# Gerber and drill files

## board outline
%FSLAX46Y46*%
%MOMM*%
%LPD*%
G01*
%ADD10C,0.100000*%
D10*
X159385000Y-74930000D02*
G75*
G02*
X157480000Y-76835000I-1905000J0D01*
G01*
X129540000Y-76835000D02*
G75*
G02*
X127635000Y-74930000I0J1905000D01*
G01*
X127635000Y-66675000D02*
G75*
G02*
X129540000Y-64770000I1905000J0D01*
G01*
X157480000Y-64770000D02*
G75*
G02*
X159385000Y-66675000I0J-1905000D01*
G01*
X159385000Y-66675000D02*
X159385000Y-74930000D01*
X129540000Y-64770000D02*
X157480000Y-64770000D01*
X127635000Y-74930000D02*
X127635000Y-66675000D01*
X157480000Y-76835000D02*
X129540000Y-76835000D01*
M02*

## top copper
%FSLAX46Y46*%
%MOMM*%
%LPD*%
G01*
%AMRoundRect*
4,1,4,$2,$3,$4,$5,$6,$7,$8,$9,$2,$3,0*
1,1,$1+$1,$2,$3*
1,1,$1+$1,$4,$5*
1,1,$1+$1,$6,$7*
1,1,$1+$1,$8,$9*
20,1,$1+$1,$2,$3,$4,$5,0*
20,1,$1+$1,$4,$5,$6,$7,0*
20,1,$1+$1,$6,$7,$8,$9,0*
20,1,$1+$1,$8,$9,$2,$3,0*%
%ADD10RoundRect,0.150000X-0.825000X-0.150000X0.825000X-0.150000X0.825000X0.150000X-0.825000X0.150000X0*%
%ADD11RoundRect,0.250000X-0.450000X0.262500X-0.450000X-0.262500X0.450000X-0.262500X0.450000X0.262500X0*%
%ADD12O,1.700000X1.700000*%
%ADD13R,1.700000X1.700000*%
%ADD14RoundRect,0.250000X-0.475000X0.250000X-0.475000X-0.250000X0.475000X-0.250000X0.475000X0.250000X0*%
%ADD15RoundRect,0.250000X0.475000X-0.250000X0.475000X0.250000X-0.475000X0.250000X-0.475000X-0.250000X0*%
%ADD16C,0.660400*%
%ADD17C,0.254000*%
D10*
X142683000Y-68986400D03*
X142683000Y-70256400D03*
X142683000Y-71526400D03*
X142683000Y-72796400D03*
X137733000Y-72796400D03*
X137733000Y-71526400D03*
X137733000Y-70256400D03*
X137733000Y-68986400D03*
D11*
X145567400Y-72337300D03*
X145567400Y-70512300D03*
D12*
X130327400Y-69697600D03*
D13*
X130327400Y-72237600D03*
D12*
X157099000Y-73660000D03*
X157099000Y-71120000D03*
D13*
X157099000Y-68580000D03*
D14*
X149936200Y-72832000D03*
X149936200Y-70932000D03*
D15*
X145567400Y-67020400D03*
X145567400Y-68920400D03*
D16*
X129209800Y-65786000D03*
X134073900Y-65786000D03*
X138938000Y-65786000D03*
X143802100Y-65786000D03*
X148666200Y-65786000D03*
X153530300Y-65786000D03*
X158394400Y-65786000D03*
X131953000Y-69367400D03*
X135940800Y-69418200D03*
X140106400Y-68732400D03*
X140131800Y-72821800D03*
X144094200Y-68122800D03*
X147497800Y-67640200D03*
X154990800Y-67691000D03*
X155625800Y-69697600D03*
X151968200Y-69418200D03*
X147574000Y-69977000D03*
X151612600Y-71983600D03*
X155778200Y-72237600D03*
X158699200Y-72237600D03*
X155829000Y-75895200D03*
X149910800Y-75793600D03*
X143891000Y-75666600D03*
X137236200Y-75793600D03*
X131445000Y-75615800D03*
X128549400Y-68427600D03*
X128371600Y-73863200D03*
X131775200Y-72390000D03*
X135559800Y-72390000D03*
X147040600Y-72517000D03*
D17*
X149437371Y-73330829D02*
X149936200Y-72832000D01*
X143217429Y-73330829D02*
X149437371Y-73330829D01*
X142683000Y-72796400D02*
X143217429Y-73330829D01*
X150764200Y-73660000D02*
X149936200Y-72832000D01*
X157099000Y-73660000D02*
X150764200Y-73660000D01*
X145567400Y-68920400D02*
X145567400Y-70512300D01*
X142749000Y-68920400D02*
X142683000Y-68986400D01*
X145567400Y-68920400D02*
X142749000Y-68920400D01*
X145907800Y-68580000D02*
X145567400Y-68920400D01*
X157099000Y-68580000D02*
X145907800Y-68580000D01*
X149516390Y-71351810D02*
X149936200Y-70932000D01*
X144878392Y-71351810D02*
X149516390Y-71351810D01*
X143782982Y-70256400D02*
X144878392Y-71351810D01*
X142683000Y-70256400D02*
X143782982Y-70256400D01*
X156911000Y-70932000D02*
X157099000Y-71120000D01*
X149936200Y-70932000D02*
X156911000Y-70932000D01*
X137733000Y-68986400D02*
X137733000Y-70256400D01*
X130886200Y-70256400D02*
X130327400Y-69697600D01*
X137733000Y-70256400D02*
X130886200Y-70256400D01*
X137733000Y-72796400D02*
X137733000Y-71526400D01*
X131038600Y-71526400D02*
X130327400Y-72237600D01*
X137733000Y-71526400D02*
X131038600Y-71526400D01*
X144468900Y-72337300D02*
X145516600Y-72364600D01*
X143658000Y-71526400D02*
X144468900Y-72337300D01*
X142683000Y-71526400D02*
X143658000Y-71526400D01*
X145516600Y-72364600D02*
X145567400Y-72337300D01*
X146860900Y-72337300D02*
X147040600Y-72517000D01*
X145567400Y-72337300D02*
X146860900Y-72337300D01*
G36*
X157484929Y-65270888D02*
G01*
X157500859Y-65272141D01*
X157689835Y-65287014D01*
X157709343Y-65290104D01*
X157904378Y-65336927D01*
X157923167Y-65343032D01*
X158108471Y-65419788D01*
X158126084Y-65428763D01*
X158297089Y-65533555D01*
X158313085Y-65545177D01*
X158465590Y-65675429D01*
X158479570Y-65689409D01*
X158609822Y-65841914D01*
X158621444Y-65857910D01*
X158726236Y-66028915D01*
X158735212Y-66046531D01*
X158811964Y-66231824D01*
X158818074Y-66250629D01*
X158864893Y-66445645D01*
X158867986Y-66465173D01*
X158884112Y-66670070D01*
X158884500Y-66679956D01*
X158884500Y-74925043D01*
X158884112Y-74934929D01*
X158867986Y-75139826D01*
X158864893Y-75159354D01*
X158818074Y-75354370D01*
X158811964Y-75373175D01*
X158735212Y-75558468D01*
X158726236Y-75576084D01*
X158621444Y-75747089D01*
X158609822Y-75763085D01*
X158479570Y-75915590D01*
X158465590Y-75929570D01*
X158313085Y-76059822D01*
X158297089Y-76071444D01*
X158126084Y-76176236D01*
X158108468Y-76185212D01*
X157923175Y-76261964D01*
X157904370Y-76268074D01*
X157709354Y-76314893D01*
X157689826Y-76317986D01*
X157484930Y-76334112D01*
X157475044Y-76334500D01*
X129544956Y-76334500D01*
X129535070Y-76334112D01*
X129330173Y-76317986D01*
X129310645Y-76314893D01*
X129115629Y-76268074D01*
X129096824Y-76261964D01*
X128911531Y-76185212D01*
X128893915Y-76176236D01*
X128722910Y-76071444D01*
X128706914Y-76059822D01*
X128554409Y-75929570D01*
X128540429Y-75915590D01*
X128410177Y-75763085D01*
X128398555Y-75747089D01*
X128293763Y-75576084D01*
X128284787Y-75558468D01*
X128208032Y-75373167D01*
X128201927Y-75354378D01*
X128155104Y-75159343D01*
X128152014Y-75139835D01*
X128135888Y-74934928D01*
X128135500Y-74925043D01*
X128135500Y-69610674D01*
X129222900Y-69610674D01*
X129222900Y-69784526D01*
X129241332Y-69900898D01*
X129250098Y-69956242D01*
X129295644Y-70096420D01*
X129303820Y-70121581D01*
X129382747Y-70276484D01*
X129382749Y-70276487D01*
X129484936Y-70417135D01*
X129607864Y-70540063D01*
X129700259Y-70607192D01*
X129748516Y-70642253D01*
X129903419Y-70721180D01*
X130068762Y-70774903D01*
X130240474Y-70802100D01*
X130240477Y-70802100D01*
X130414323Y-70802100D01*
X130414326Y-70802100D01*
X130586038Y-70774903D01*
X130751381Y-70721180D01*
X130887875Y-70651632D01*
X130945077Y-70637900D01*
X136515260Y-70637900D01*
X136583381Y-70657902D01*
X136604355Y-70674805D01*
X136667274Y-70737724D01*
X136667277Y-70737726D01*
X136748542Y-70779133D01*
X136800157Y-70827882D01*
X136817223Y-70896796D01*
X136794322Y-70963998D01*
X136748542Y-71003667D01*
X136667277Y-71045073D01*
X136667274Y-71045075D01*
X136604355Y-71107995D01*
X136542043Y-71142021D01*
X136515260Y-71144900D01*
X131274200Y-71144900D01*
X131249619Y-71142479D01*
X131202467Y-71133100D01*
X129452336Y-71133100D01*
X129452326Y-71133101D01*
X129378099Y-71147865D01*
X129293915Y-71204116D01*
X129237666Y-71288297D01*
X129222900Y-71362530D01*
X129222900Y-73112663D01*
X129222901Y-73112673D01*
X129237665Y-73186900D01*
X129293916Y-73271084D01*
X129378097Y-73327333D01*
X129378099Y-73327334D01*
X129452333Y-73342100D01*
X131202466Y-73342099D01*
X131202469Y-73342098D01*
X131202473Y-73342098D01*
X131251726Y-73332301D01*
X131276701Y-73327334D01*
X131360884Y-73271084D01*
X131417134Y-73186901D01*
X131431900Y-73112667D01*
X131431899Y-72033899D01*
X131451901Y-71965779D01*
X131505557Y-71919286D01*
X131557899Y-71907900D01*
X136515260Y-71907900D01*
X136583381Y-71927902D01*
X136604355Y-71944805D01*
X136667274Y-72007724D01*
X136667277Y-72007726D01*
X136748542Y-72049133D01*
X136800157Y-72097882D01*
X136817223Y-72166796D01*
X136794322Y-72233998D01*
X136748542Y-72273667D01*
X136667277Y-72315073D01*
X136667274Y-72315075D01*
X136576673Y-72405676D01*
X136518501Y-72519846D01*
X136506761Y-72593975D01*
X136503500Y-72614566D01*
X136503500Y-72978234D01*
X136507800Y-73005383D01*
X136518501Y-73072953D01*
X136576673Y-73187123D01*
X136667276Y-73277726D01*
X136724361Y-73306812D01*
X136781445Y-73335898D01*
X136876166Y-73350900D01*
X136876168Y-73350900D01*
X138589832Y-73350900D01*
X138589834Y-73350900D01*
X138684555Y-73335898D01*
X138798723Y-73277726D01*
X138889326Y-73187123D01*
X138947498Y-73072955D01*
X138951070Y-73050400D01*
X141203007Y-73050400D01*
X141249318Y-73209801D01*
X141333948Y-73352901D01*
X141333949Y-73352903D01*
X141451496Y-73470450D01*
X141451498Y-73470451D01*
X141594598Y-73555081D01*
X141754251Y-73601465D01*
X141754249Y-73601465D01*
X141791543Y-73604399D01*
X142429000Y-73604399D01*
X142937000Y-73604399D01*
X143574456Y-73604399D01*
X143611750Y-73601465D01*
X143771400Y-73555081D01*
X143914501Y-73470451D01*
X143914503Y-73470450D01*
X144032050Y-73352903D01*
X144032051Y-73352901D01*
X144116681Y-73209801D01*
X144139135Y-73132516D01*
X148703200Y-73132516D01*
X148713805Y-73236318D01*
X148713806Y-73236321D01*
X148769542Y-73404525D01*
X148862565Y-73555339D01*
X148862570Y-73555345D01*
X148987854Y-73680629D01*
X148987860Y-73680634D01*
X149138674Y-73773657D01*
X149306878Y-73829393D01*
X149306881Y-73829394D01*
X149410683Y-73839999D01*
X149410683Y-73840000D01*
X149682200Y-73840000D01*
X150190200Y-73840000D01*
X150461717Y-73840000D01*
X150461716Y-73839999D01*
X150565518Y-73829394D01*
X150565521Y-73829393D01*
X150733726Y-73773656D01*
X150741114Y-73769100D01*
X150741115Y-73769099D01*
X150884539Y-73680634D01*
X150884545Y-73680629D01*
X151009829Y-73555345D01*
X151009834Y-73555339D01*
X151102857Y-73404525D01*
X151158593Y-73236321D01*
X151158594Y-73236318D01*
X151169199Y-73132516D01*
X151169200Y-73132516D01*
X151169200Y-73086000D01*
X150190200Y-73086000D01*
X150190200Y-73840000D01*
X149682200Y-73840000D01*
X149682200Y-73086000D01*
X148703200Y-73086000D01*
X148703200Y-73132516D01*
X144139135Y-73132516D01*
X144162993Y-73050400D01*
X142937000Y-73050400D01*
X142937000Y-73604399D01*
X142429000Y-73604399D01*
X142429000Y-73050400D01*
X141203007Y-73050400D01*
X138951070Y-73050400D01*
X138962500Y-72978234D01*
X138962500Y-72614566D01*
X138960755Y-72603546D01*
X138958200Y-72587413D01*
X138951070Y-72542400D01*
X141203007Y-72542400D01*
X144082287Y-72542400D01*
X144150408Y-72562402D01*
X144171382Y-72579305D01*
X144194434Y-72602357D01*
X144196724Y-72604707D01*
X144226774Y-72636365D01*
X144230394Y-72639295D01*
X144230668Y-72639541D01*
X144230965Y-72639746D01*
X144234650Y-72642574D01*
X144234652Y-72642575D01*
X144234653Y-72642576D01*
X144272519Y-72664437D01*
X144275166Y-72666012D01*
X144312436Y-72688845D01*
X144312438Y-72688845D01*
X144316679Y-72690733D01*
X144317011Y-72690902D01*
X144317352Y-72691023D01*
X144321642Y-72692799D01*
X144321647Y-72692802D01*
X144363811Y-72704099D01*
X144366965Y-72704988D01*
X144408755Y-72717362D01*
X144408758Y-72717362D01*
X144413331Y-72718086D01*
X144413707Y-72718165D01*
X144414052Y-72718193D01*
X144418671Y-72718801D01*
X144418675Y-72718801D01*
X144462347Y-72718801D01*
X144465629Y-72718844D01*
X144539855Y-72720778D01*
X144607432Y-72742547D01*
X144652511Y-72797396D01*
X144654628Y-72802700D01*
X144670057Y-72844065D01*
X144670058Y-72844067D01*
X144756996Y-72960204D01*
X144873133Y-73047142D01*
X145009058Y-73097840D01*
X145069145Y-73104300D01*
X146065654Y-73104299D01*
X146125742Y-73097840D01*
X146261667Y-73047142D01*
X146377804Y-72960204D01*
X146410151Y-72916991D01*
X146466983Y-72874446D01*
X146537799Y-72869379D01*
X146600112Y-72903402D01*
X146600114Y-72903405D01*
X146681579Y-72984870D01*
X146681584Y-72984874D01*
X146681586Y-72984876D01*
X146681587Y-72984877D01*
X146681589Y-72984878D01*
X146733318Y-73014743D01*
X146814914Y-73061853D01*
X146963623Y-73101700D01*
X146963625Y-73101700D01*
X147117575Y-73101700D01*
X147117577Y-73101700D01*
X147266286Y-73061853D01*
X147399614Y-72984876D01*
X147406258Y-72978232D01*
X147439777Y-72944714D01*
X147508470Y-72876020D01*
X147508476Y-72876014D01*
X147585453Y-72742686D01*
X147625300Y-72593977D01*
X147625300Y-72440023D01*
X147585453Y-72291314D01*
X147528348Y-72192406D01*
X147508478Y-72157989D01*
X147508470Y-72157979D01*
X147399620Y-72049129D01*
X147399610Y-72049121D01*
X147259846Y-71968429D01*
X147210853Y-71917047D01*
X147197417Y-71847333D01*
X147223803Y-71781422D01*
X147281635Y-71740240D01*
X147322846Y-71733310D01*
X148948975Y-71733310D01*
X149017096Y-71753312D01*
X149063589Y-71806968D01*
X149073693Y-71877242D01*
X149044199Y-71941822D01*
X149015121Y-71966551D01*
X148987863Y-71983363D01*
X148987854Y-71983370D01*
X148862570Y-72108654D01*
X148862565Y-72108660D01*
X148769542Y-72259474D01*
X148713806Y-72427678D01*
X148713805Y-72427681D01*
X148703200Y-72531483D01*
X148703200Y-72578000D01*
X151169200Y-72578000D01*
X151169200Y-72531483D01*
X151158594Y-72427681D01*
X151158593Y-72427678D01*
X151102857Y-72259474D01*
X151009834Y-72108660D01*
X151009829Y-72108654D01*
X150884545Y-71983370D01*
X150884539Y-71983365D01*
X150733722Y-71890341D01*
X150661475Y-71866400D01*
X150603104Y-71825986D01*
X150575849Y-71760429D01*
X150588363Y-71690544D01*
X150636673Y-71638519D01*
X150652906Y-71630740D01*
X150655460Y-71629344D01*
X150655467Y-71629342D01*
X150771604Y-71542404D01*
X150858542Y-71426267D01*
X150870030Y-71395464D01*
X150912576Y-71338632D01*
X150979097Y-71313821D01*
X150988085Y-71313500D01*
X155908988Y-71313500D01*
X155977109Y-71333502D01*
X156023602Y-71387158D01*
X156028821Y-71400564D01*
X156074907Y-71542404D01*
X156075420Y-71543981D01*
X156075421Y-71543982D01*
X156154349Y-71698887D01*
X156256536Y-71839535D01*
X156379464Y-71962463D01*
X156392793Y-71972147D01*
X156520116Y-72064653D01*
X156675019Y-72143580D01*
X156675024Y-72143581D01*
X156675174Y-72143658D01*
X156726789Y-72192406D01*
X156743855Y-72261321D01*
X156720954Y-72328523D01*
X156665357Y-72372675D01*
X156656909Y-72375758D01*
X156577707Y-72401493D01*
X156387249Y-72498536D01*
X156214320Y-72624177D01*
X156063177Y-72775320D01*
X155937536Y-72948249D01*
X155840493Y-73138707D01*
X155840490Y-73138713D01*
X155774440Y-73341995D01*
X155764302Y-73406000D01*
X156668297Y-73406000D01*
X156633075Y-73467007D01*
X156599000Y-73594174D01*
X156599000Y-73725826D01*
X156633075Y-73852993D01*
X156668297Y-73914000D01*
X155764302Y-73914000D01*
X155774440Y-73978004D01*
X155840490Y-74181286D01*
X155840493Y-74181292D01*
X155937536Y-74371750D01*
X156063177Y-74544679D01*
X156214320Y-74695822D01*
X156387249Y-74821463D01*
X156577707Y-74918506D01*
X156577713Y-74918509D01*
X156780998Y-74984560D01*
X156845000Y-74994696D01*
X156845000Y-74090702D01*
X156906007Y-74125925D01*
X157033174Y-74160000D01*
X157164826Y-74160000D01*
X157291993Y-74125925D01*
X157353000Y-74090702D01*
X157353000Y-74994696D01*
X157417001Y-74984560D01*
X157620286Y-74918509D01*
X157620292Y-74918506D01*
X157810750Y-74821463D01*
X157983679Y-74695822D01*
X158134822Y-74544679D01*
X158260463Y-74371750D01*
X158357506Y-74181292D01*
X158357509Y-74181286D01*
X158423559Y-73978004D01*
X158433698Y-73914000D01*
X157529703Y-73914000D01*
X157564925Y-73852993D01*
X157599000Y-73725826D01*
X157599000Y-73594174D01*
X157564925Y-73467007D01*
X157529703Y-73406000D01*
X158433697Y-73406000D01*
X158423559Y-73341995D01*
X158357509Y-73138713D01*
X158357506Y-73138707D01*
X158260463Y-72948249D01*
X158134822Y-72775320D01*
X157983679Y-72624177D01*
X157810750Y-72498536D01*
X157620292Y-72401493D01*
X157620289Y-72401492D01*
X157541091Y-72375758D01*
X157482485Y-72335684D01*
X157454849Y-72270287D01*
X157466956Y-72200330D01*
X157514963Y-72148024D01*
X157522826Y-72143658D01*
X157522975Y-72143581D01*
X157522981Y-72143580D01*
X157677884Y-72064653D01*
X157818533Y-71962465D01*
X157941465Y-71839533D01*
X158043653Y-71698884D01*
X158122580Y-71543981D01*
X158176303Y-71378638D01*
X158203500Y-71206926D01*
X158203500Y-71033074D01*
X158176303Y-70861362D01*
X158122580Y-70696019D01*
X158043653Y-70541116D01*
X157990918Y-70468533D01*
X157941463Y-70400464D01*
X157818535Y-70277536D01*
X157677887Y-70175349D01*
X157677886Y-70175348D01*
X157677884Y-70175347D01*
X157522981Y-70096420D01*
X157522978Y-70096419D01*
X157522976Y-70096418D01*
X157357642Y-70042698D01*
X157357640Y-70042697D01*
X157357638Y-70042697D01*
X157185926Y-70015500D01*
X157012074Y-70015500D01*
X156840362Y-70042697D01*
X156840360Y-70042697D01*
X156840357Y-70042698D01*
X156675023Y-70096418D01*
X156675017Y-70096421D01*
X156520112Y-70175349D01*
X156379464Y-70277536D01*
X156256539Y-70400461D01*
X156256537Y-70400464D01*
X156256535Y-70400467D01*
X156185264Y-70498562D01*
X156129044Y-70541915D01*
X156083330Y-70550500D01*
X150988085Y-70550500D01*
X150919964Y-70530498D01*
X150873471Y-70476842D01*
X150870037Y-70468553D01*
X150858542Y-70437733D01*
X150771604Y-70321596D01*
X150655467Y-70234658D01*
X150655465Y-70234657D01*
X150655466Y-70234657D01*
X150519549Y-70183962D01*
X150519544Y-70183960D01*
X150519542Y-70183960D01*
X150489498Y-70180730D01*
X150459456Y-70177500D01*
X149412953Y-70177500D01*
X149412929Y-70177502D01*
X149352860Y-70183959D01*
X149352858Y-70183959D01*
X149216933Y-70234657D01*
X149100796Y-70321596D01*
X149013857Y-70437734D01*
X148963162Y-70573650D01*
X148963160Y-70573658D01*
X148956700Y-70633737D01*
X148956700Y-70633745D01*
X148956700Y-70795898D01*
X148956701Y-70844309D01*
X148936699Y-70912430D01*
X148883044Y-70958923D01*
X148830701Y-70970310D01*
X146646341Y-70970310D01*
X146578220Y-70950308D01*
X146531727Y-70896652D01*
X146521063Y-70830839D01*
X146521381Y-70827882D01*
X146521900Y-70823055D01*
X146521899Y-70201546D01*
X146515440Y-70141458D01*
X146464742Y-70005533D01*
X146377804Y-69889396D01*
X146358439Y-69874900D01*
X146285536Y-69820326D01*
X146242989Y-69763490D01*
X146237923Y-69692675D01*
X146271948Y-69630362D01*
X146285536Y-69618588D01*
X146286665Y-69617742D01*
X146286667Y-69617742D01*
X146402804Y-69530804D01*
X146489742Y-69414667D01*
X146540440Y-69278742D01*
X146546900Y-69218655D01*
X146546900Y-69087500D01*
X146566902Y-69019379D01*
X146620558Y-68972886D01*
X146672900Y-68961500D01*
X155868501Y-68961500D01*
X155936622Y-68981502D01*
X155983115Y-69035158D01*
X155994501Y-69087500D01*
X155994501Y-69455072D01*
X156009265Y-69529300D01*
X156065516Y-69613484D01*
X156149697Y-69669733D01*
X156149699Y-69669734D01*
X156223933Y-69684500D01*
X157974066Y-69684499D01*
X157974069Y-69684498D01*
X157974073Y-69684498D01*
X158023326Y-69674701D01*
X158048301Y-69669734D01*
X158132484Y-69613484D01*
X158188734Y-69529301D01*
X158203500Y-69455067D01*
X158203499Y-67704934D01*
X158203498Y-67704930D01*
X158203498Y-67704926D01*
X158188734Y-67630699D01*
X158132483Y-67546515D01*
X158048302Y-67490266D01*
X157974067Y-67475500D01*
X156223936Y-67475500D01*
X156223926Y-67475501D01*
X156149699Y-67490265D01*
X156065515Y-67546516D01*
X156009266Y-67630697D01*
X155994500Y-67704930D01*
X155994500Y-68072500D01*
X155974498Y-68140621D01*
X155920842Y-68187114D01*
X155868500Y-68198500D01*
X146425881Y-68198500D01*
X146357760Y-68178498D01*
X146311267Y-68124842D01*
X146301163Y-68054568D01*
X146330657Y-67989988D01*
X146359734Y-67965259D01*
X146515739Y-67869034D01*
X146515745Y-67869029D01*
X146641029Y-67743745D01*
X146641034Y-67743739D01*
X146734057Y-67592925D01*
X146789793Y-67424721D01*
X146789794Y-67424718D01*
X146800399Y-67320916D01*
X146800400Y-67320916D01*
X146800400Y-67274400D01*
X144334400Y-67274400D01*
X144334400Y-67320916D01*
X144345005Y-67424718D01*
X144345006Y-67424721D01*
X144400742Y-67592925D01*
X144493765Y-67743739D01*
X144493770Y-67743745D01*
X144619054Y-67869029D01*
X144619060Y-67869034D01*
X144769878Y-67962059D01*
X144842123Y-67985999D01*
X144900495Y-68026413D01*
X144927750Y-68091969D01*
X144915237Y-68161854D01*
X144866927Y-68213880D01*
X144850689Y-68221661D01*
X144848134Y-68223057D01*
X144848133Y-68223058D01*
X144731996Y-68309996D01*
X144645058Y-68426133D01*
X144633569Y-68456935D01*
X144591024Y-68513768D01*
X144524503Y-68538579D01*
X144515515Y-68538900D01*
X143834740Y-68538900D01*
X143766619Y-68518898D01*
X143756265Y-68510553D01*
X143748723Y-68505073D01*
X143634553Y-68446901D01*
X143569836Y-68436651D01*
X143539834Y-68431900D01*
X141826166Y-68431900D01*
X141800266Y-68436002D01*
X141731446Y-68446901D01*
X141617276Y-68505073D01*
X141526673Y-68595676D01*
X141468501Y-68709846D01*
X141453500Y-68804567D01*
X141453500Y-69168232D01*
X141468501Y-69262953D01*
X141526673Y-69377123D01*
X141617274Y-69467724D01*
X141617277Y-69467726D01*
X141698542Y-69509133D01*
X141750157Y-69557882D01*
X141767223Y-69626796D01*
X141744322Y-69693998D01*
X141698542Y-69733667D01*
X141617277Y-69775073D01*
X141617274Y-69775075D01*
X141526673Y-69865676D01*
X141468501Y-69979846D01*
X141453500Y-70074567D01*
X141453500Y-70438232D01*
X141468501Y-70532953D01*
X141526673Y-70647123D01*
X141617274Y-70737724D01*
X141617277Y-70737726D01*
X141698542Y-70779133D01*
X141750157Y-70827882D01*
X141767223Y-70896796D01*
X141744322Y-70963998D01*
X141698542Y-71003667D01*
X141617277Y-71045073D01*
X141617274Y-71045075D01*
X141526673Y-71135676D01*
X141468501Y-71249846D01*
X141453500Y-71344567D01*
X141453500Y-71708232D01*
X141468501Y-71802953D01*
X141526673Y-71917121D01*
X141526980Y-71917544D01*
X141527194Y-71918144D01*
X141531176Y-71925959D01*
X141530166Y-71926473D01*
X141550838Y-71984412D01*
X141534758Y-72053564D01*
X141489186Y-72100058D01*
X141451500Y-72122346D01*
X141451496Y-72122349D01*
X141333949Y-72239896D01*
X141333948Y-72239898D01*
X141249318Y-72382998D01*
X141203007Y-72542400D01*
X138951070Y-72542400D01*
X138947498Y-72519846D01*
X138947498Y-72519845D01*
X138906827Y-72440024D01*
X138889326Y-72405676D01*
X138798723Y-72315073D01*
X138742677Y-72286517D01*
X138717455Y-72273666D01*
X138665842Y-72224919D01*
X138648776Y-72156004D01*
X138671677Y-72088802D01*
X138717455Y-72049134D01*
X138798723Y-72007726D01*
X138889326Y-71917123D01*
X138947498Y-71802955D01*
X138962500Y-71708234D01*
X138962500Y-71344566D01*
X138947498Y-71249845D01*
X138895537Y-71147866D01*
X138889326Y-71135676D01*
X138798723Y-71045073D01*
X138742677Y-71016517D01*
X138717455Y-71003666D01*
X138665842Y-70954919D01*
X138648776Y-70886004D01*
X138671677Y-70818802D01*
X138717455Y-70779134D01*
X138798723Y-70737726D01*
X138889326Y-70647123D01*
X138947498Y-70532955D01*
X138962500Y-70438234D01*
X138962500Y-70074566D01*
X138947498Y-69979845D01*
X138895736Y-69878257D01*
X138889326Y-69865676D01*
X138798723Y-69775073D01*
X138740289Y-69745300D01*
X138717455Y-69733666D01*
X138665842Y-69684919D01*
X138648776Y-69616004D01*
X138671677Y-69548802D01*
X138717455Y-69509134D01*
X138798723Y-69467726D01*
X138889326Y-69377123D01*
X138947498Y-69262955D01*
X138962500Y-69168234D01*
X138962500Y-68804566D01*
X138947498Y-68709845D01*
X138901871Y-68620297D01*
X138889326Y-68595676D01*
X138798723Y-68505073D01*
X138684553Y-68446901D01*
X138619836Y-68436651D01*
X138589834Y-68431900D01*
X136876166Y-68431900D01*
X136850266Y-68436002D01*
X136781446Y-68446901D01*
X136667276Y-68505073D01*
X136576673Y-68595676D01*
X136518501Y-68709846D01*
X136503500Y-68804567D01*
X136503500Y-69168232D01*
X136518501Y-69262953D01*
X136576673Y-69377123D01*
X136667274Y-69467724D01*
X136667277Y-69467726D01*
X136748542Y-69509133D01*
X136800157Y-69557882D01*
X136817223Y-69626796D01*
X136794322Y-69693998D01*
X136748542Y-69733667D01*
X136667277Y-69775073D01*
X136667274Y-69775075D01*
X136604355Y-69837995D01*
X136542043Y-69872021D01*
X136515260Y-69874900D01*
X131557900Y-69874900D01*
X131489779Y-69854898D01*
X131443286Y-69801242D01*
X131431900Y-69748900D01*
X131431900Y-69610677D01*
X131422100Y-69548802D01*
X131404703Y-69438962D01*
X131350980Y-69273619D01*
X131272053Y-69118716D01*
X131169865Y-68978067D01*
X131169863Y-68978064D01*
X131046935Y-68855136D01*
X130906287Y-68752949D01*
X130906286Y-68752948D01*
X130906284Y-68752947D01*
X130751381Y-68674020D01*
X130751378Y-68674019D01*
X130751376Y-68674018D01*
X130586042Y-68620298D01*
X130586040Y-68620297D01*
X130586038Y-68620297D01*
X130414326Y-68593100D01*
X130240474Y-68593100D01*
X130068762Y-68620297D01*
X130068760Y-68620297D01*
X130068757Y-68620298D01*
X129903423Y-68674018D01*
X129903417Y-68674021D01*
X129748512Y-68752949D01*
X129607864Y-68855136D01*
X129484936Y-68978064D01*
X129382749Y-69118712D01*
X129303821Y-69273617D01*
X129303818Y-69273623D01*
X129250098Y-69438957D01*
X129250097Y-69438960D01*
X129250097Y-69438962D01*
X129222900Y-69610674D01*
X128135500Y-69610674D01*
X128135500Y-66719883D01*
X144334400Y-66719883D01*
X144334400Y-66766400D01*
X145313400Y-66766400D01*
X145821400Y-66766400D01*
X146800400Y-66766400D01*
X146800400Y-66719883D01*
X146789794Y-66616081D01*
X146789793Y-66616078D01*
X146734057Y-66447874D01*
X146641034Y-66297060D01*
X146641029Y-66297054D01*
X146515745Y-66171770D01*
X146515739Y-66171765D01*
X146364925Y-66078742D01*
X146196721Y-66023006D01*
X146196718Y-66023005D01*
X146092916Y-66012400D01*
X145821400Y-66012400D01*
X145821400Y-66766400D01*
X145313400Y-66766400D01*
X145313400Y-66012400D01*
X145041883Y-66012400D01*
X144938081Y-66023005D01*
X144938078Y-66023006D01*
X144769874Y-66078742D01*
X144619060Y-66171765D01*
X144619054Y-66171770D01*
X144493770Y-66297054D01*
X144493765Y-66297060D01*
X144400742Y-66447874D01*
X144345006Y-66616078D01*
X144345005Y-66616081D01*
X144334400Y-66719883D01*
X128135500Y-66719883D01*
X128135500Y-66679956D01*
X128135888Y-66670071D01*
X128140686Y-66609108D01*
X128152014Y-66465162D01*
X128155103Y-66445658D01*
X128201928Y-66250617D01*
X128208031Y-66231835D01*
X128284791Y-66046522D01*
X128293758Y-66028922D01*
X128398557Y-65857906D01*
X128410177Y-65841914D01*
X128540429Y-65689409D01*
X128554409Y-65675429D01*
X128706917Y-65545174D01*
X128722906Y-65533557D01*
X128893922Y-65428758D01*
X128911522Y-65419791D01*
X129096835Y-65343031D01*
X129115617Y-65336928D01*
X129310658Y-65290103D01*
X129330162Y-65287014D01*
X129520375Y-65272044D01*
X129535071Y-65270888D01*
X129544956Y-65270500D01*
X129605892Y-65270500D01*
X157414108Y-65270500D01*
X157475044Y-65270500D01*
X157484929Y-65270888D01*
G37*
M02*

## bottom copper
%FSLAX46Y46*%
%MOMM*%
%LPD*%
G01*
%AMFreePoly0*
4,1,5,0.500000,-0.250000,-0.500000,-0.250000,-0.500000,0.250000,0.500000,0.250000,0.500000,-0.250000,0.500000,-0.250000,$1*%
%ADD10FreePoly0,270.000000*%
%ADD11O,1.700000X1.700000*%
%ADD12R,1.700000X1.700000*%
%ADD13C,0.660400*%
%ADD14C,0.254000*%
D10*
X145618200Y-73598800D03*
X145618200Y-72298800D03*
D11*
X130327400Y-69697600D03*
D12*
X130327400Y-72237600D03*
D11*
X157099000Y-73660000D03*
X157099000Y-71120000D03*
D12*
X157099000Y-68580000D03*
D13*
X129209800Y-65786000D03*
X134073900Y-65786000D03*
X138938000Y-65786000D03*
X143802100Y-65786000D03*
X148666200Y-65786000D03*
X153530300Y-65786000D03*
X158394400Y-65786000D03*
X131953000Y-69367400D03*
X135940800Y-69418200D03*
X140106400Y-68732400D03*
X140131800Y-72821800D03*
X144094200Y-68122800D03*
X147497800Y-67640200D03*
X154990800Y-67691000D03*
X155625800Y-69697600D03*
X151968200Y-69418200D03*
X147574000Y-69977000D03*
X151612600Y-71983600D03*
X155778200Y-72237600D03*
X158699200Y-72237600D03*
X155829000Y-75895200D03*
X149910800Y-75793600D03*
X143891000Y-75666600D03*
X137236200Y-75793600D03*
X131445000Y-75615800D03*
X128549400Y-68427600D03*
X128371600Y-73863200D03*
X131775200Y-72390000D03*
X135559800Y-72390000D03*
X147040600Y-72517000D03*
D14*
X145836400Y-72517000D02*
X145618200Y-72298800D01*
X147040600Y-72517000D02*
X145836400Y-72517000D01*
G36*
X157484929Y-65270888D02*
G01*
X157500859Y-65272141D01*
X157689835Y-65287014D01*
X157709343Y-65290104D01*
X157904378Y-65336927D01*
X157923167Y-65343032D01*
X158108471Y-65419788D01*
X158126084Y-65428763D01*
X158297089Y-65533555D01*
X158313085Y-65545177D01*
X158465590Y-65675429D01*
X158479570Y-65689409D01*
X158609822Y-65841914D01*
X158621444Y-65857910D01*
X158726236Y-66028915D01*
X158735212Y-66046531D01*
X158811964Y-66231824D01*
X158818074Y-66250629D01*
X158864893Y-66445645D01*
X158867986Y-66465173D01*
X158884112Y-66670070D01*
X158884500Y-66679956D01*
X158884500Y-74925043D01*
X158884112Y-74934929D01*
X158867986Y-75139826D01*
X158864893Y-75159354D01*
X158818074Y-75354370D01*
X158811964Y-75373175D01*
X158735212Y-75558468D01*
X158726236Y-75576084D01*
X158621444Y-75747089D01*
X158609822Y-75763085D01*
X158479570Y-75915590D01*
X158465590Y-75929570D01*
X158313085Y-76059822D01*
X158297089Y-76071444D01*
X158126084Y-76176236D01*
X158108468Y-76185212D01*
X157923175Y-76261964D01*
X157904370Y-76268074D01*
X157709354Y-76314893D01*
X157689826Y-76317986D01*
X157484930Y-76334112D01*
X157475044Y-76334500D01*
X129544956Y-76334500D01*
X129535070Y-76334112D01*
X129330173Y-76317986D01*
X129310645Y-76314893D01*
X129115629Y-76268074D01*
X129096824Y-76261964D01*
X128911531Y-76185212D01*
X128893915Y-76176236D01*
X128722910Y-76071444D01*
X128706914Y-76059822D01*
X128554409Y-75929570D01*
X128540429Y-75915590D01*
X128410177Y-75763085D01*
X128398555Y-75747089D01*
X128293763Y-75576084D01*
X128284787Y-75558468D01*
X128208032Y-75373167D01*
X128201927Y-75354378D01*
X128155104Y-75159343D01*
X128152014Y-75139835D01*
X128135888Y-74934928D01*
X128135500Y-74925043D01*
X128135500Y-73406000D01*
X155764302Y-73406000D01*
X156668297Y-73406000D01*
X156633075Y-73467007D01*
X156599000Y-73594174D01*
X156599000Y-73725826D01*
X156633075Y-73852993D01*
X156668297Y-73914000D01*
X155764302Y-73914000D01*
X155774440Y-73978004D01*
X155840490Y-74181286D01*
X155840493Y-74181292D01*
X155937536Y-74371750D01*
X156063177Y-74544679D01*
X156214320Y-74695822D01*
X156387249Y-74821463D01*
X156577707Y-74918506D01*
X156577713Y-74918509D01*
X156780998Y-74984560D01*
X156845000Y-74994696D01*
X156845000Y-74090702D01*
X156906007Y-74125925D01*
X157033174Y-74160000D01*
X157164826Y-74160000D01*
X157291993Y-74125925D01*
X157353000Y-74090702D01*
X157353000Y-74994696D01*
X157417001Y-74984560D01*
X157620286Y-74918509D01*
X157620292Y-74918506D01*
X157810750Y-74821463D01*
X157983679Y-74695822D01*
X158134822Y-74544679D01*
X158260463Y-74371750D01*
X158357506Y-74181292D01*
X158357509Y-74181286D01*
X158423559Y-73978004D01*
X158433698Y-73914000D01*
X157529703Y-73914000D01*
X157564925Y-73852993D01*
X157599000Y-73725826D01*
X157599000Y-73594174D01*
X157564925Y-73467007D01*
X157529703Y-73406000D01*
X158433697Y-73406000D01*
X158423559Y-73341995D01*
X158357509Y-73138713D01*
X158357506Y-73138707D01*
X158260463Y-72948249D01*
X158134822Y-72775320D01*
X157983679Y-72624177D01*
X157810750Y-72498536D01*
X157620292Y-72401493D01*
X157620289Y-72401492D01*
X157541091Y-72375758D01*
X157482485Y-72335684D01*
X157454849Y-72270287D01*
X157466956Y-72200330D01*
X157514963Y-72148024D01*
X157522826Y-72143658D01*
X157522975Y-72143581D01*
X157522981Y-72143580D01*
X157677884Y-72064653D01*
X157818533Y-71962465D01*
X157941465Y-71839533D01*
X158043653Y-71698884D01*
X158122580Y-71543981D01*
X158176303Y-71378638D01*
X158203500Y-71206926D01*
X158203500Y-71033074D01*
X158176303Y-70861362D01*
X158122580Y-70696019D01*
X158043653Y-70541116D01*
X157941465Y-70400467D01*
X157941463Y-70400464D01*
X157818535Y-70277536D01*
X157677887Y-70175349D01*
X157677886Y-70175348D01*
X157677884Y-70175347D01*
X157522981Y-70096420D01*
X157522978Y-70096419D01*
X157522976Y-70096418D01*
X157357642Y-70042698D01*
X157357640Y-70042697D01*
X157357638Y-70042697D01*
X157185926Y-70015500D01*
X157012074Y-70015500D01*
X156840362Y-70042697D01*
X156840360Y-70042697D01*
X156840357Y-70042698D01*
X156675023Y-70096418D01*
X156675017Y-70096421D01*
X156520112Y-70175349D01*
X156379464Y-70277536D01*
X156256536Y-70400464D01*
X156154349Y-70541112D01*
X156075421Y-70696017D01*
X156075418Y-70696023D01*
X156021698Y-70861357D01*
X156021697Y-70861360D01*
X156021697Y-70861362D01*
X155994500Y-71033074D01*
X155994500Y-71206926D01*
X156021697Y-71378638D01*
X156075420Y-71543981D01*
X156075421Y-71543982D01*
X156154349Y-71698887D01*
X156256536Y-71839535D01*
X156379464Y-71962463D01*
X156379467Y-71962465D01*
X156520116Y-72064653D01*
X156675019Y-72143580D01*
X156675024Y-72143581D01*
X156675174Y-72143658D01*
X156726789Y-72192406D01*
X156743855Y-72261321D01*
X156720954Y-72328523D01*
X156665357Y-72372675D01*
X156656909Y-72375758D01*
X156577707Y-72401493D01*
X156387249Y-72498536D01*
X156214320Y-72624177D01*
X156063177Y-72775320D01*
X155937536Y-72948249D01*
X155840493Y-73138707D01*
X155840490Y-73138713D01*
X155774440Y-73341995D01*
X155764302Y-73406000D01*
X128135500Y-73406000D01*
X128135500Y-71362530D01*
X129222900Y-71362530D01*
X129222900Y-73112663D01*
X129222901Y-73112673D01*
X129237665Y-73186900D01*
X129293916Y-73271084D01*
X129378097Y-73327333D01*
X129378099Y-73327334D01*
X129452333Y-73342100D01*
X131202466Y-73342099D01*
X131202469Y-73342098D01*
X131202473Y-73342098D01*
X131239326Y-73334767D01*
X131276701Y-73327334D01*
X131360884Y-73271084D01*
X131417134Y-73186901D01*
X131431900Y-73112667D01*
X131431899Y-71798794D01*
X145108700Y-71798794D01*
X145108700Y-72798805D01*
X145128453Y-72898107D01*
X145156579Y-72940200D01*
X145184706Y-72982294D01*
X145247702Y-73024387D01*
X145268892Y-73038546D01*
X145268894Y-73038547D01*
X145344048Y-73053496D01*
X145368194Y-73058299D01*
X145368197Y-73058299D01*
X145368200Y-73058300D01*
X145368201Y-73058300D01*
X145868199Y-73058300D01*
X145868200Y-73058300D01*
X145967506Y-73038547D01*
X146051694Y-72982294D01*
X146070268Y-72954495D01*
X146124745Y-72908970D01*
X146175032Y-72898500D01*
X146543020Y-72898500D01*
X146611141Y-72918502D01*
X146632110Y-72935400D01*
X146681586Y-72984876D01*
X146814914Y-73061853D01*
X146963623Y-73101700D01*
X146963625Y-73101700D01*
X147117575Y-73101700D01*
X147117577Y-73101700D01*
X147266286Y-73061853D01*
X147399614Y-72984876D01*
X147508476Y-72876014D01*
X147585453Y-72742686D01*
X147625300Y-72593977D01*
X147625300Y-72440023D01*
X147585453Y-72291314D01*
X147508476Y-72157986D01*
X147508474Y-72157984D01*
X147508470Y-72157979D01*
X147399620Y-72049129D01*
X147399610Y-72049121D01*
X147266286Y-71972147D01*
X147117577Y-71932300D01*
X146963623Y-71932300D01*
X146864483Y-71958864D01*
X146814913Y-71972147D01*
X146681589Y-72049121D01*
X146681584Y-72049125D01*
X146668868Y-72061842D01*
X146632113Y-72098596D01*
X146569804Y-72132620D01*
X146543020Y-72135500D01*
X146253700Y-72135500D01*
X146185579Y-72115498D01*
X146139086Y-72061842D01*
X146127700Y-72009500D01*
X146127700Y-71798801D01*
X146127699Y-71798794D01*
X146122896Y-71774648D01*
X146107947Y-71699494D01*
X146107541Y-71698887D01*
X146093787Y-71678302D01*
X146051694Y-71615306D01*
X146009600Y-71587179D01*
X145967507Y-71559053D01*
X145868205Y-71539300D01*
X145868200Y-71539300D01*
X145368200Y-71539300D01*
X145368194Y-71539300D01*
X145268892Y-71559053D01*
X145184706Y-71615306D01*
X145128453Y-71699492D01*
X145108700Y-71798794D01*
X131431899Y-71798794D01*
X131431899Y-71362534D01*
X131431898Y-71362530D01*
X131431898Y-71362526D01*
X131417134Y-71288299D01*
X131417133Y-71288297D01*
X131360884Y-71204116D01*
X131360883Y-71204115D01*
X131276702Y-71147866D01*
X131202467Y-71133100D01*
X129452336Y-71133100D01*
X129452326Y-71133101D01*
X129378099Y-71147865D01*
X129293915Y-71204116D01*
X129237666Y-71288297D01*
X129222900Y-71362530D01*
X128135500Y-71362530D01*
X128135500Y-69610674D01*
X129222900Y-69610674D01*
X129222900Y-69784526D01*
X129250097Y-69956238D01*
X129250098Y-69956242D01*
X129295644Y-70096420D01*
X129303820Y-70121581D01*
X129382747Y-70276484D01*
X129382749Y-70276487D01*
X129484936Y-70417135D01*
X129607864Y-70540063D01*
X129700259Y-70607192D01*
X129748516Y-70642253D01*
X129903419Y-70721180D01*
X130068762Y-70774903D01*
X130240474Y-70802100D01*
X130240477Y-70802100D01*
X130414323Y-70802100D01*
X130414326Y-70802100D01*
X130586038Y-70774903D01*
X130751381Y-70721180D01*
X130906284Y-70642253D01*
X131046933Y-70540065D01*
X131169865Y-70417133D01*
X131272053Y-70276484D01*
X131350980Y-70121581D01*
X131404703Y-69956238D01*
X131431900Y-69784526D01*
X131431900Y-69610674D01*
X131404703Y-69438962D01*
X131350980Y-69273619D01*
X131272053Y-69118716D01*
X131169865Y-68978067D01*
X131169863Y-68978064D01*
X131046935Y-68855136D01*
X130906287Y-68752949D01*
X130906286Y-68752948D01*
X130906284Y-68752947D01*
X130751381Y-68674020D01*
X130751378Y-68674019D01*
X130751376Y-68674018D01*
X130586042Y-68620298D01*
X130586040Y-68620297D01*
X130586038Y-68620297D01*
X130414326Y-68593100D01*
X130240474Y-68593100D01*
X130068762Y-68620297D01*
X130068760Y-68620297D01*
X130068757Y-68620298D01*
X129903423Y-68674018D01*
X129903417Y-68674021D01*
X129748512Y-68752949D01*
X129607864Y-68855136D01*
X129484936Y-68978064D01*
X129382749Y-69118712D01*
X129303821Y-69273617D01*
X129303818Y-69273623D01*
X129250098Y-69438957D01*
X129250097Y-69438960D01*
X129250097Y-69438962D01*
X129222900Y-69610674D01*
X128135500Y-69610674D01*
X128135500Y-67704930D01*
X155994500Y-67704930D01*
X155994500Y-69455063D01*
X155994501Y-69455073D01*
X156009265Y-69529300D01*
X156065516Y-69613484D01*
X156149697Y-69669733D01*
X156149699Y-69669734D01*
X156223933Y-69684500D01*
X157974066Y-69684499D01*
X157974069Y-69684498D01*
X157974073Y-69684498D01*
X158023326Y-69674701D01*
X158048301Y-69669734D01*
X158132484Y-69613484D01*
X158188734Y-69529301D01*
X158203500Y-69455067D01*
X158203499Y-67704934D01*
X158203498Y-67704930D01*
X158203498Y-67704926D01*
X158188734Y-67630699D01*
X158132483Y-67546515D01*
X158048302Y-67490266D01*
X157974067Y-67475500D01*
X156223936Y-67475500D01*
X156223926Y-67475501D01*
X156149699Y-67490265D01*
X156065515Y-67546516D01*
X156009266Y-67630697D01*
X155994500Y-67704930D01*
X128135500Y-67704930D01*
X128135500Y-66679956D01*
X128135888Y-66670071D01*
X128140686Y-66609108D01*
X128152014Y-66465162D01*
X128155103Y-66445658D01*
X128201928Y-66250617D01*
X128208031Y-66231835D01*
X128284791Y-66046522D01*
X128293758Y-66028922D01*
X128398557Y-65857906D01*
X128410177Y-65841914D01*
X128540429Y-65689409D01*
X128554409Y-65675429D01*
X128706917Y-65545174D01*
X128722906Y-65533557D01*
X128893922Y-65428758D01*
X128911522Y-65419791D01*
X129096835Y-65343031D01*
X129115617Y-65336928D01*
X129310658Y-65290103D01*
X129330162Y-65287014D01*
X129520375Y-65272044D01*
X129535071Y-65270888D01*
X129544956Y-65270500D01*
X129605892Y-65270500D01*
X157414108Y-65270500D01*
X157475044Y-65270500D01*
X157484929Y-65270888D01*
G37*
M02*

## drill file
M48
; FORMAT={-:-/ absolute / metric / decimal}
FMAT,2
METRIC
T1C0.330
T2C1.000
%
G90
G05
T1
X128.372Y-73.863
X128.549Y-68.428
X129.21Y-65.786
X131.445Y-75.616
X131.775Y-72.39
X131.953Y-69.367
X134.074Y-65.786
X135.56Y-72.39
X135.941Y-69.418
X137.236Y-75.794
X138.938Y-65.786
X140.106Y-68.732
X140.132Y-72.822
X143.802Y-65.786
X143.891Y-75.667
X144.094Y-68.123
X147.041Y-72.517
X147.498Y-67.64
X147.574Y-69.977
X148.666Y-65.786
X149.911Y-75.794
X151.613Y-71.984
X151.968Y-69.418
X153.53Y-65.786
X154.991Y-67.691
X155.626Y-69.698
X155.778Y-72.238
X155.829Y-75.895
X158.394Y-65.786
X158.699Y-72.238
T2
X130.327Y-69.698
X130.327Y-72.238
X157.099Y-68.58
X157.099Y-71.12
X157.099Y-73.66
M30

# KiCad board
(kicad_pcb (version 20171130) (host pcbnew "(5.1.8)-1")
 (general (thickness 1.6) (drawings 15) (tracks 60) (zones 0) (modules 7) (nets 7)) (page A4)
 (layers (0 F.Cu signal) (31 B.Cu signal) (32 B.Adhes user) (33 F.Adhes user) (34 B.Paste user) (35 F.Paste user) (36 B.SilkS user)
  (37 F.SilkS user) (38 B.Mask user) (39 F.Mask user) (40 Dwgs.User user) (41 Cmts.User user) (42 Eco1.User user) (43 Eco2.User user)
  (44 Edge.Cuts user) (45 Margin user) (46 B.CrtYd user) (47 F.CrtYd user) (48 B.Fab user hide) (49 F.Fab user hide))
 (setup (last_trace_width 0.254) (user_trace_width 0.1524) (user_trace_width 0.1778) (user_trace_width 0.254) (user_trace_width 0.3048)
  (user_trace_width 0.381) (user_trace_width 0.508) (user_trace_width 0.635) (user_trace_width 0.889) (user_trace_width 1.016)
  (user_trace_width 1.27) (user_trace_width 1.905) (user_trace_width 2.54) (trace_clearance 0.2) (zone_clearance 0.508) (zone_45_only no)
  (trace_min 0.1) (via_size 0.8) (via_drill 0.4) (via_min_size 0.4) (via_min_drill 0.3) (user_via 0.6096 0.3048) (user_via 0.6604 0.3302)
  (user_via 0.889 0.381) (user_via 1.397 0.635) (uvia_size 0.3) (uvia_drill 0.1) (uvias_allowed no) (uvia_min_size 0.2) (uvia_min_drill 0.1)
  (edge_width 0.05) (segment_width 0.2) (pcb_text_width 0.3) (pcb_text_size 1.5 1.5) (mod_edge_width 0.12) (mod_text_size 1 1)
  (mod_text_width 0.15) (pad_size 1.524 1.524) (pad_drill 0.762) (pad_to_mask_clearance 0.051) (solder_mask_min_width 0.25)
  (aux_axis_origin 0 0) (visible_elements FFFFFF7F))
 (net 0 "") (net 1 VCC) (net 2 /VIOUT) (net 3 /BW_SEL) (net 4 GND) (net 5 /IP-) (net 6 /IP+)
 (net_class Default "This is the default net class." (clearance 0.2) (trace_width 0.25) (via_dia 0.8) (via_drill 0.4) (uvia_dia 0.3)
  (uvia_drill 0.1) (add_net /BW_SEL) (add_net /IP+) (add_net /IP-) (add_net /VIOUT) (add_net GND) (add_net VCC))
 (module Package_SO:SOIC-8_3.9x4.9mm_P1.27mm (layer F.Cu) (at 140.208 70.8914)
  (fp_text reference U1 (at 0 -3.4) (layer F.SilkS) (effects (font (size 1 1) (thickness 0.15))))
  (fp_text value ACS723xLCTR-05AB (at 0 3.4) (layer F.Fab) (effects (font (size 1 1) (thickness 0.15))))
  (pad 8 smd roundrect (at 2.475 -1.905) (size 1.95 0.6) (layers F.Cu F.Paste F.Mask) (roundrect_rratio 0.25) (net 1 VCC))
  (pad 7 smd roundrect (at 2.475 -0.635) (size 1.95 0.6) (layers F.Cu F.Paste F.Mask) (roundrect_rratio 0.25) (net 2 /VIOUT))
  (pad 6 smd roundrect (at 2.475 0.635) (size 1.95 0.6) (layers F.Cu F.Paste F.Mask) (roundrect_rratio 0.25) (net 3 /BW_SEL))
  (pad 5 smd roundrect (at 2.475 1.905) (size 1.95 0.6) (layers F.Cu F.Paste F.Mask) (roundrect_rratio 0.25) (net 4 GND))
  (pad 4 smd roundrect (at -2.475 1.905) (size 1.95 0.6) (layers F.Cu F.Paste F.Mask) (roundrect_rratio 0.25) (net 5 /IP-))
  (pad 3 smd roundrect (at -2.475 0.635) (size 1.95 0.6) (layers F.Cu F.Paste F.Mask) (roundrect_rratio 0.25) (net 5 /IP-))
  (pad 2 smd roundrect (at -2.475 -0.635) (size 1.95 0.6) (layers F.Cu F.Paste F.Mask) (roundrect_rratio 0.25) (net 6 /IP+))
  (pad 1 smd roundrect (at -2.475 -1.905) (size 1.95 0.6) (layers F.Cu F.Paste F.Mask) (roundrect_rratio 0.25) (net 6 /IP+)))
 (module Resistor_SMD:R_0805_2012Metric (layer F.Cu) (at 145.5674 71.4248 270)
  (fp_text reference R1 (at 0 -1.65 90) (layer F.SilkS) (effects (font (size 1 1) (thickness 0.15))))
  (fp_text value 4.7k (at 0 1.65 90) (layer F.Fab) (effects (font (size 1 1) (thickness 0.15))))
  (pad 2 smd roundrect (at 0.9125 0 270) (size 1.025 1.4) (layers F.Cu F.Paste F.Mask) (roundrect_rratio 0.243902) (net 3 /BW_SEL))
  (pad 1 smd roundrect (at -0.9125 0 270) (size 1.025 1.4) (layers F.Cu F.Paste F.Mask) (roundrect_rratio 0.243902) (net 1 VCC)))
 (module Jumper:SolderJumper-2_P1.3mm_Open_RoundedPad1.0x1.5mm (layer B.Cu) (at 145.6182 72.9488 270)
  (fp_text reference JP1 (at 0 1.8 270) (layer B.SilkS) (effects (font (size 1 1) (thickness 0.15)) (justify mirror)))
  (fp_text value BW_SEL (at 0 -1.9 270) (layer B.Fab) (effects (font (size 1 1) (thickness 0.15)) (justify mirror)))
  (pad 2 smd custom (at 0.65 0 270) (size 1 0.5) (layers B.Cu B.Mask) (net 4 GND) (zone_connect 2)
   (options (clearance outline) (anchor rect)) (primitives))
  (pad 1 smd custom (at -0.65 0 270) (size 1 0.5) (layers B.Cu B.Mask) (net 3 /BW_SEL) (zone_connect 2)
   (options (clearance outline) (anchor rect)) (primitives)))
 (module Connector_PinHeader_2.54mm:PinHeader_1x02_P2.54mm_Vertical (layer F.Cu) (at 130.3274 72.2376 180)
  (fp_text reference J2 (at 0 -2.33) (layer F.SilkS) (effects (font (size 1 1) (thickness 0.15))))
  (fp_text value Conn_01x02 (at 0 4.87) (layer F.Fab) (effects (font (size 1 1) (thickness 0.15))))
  (pad 2 thru_hole oval (at 0 2.54 180) (size 1.7 1.7) (drill 1) (layers *.Cu *.Mask) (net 6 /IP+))
  (pad 1 thru_hole rect (at 0 0 180) (size 1.7 1.7) (drill 1) (layers *.Cu *.Mask) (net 5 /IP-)))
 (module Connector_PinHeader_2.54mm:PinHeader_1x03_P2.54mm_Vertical (layer F.Cu) (at 157.099 68.58)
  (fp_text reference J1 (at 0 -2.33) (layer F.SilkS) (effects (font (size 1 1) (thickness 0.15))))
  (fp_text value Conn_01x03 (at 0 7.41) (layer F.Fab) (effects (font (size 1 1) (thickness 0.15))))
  (pad 3 thru_hole oval (at 0 5.08) (size 1.7 1.7) (drill 1) (layers *.Cu *.Mask) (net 4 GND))
  (pad 2 thru_hole oval (at 0 2.54) (size 1.7 1.7) (drill 1) (layers *.Cu *.Mask) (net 2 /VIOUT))
  (pad 1 thru_hole rect (at 0 0) (size 1.7 1.7) (drill 1) (layers *.Cu *.Mask) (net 1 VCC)))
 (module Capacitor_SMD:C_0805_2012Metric (layer F.Cu) (at 149.9362 71.882 270)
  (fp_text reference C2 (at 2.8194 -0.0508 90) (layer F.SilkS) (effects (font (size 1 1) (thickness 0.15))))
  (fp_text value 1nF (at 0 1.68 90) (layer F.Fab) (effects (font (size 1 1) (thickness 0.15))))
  (pad 2 smd roundrect (at 0.95 0 270) (size 1 1.45) (layers F.Cu F.Paste F.Mask) (roundrect_rratio 0.25) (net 4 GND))
  (pad 1 smd roundrect (at -0.95 0 270) (size 1 1.45) (layers F.Cu F.Paste F.Mask) (roundrect_rratio 0.25) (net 2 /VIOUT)))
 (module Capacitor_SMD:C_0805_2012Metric (layer F.Cu) (at 145.5674 67.9704 90)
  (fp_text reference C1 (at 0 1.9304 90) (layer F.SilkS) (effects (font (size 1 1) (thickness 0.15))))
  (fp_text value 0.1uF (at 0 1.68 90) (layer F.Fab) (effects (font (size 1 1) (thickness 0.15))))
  (pad 2 smd roundrect (at 0.95 0 90) (size 1 1.45) (layers F.Cu F.Paste F.Mask) (roundrect_rratio 0.25) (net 4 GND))
  (pad 1 smd roundrect (at -0.95 0 90) (size 1 1.45) (layers F.Cu F.Paste F.Mask) (roundrect_rratio 0.25) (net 1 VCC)))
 (gr_arc (start 157.48 74.93) (end 157.48 76.835) (angle -90) (layer Edge.Cuts) (width 0.1))
 (gr_arc (start 129.54 74.93) (end 127.635 74.93) (angle -90) (layer Edge.Cuts) (width 0.1))
 (gr_arc (start 129.54 66.675) (end 129.54 64.77) (angle -90) (layer Edge.Cuts) (width 0.1))
 (gr_arc (start 157.48 66.675) (end 159.385 66.675) (angle -90) (layer Edge.Cuts) (width 0.1))
 (gr_line (start 159.385 66.675) (end 159.385 74.93) (layer Edge.Cuts) (width 0.1))
 (gr_line (start 129.54 64.77) (end 157.48 64.77) (layer Edge.Cuts) (width 0.1))
 (gr_line (start 127.635 74.93) (end 127.635 66.675) (layer Edge.Cuts) (width 0.1))
 (gr_line (start 157.48 76.835) (end 129.54 76.835) (layer Edge.Cuts) (width 0.1))
 (segment (start 149.437371 73.330829) (end 149.9362 72.832) (width 0.254) (layer F.Cu) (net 4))
 (segment (start 143.217429 73.330829) (end 149.437371 73.330829) (width 0.254) (layer F.Cu) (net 4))
 (segment (start 142.683 72.7964) (end 143.217429 73.330829) (width 0.254) (layer F.Cu) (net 4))
 (segment (start 150.7642 73.66) (end 149.9362 72.832) (width 0.254) (layer F.Cu) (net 4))
 (segment (start 157.099 73.66) (end 150.7642 73.66) (width 0.254) (layer F.Cu) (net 4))
 (via (at 129.2098 65.786) (size 0.6604) (drill 0.3302) (layers F.Cu B.Cu) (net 4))
 (via (at 134.0739 65.786) (size 0.6604) (drill 0.3302) (layers F.Cu B.Cu) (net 4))
 (via (at 138.938 65.786) (size 0.6604) (drill 0.3302) (layers F.Cu B.Cu) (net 4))
 (via (at 143.8021 65.786) (size 0.6604) (drill 0.3302) (layers F.Cu B.Cu) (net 4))
 (via (at 148.6662 65.786) (size 0.6604) (drill 0.3302) (layers F.Cu B.Cu) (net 4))
 (via (at 153.5303 65.786) (size 0.6604) (drill 0.3302) (layers F.Cu B.Cu) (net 4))
 (via (at 158.3944 65.786) (size 0.6604) (drill 0.3302) (layers F.Cu B.Cu) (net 4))
 (via (at 131.953 69.3674) (size 0.6604) (drill 0.3302) (layers F.Cu B.Cu) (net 4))
 (via (at 135.9408 69.4182) (size 0.6604) (drill 0.3302) (layers F.Cu B.Cu) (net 4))
 (via (at 140.1064 68.7324) (size 0.6604) (drill 0.3302) (layers F.Cu B.Cu) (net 4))
 (via (at 140.1318 72.8218) (size 0.6604) (drill 0.3302) (layers F.Cu B.Cu) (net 4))
 (via (at 144.0942 68.1228) (size 0.6604) (drill 0.3302) (layers F.Cu B.Cu) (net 4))
 (via (at 147.4978 67.6402) (size 0.6604) (drill 0.3302) (layers F.Cu B.Cu) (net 4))
 (via (at 154.9908 67.691) (size 0.6604) (drill 0.3302) (layers F.Cu B.Cu) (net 4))
 (via (at 155.6258 69.6976) (size 0.6604) (drill 0.3302) (layers F.Cu B.Cu) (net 4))
 (via (at 151.9682 69.4182) (size 0.6604) (drill 0.3302) (layers F.Cu B.Cu) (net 4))
 (via (at 147.574 69.977) (size 0.6604) (drill 0.3302) (layers F.Cu B.Cu) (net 4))
 (via (at 151.6126 71.9836) (size 0.6604) (drill 0.3302) (layers F.Cu B.Cu) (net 4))
 (via (at 155.7782 72.2376) (size 0.6604) (drill 0.3302) (layers F.Cu B.Cu) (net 4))
 (via (at 158.6992 72.2376) (size 0.6604) (drill 0.3302) (layers F.Cu B.Cu) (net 4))
 (via (at 155.829 75.8952) (size 0.6604) (drill 0.3302) (layers F.Cu B.Cu) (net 4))
 (via (at 149.9108 75.7936) (size 0.6604) (drill 0.3302) (layers F.Cu B.Cu) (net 4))
 (via (at 143.891 75.6666) (size 0.6604) (drill 0.3302) (layers F.Cu B.Cu) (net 4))
 (via (at 137.2362 75.7936) (size 0.6604) (drill 0.3302) (layers F.Cu B.Cu) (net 4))
 (via (at 131.445 75.6158) (size 0.6604) (drill 0.3302) (layers F.Cu B.Cu) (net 4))
 (via (at 128.5494 68.4276) (size 0.6604) (drill 0.3302) (layers F.Cu B.Cu) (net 4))
 (via (at 128.3716 73.8632) (size 0.6604) (drill 0.3302) (layers F.Cu B.Cu) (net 4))
 (via (at 131.7752 72.39) (size 0.6604) (drill 0.3302) (layers F.Cu B.Cu) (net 4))
 (via (at 135.5598 72.39) (size 0.6604) (drill 0.3302) (layers F.Cu B.Cu) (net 4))
 (segment (start 145.5674 68.9204) (end 145.5674 70.5123) (width 0.254) (layer F.Cu) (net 1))
 (segment (start 142.749 68.9204) (end 142.683 68.9864) (width 0.254) (layer F.Cu) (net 1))
 (segment (start 145.5674 68.9204) (end 142.749 68.9204) (width 0.254) (layer F.Cu) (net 1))
 (segment (start 145.9078 68.58) (end 145.5674 68.9204) (width 0.254) (layer F.Cu) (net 1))
 (segment (start 157.099 68.58) (end 145.9078 68.58) (width 0.254) (layer F.Cu) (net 1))
 (segment (start 149.51639 71.35181) (end 149.9362 70.932) (width 0.254) (layer F.Cu) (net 2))
 (segment (start 144.878392 71.35181) (end 149.51639 71.35181) (width 0.254) (layer F.Cu) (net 2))
 (segment (start 143.782982 70.2564) (end 144.878392 71.35181) (width 0.254) (layer F.Cu) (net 2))
 (segment (start 142.683 70.2564) (end 143.782982 70.2564) (width 0.254) (layer F.Cu) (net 2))
 (segment (start 156.911 70.932) (end 157.099 71.12) (width 0.254) (layer F.Cu) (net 2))
 (segment (start 149.9362 70.932) (end 156.911 70.932) (width 0.254) (layer F.Cu) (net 2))
 (segment (start 137.733 68.9864) (end 137.733 70.2564) (width 0.254) (layer F.Cu) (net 6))
 (segment (start 130.8862 70.2564) (end 130.3274 69.6976) (width 0.254) (layer F.Cu) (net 6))
 (segment (start 137.733 70.2564) (end 130.8862 70.2564) (width 0.254) (layer F.Cu) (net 6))
 (segment (start 137.733 72.7964) (end 137.733 71.5264) (width 0.254) (layer F.Cu) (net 5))
 (segment (start 131.0386 71.5264) (end 130.3274 72.2376) (width 0.254) (layer F.Cu) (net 5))
 (segment (start 137.733 71.5264) (end 131.0386 71.5264) (width 0.254) (layer F.Cu) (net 5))
 (segment (start 144.4689 72.3373) (end 145.5166 72.3646) (width 0.254) (layer F.Cu) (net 3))
 (segment (start 143.658 71.5264) (end 144.4689 72.3373) (width 0.254) (layer F.Cu) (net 3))
 (segment (start 142.683 71.5264) (end 143.658 71.5264) (width 0.254) (layer F.Cu) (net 3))
 (segment (start 145.5166 72.3646) (end 145.5674 72.3373) (width 0.254) (layer F.Cu) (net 3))
 (via (at 147.0406 72.517) (size 0.6604) (drill 0.3302) (layers F.Cu B.Cu) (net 3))
 (segment (start 146.8609 72.3373) (end 147.0406 72.517) (width 0.254) (layer F.Cu) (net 3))
 (segment (start 145.5674 72.3373) (end 146.8609 72.3373) (width 0.254) (layer F.Cu) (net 3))
 (segment (start 145.8364 72.517) (end 145.6182 72.2988) (width 0.254) (layer B.Cu) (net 3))
 (segment (start 147.0406 72.517) (end 145.8364 72.517) (width 0.254) (layer B.Cu) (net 3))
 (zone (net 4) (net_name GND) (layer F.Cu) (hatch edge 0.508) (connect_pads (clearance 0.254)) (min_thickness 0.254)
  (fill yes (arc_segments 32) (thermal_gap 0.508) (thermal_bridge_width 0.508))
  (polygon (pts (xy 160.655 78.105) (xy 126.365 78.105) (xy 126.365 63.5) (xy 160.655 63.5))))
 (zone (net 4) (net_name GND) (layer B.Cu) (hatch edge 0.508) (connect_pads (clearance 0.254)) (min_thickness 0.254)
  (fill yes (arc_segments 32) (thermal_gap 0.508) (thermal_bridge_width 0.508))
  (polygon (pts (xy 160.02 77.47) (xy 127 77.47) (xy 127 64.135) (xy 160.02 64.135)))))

